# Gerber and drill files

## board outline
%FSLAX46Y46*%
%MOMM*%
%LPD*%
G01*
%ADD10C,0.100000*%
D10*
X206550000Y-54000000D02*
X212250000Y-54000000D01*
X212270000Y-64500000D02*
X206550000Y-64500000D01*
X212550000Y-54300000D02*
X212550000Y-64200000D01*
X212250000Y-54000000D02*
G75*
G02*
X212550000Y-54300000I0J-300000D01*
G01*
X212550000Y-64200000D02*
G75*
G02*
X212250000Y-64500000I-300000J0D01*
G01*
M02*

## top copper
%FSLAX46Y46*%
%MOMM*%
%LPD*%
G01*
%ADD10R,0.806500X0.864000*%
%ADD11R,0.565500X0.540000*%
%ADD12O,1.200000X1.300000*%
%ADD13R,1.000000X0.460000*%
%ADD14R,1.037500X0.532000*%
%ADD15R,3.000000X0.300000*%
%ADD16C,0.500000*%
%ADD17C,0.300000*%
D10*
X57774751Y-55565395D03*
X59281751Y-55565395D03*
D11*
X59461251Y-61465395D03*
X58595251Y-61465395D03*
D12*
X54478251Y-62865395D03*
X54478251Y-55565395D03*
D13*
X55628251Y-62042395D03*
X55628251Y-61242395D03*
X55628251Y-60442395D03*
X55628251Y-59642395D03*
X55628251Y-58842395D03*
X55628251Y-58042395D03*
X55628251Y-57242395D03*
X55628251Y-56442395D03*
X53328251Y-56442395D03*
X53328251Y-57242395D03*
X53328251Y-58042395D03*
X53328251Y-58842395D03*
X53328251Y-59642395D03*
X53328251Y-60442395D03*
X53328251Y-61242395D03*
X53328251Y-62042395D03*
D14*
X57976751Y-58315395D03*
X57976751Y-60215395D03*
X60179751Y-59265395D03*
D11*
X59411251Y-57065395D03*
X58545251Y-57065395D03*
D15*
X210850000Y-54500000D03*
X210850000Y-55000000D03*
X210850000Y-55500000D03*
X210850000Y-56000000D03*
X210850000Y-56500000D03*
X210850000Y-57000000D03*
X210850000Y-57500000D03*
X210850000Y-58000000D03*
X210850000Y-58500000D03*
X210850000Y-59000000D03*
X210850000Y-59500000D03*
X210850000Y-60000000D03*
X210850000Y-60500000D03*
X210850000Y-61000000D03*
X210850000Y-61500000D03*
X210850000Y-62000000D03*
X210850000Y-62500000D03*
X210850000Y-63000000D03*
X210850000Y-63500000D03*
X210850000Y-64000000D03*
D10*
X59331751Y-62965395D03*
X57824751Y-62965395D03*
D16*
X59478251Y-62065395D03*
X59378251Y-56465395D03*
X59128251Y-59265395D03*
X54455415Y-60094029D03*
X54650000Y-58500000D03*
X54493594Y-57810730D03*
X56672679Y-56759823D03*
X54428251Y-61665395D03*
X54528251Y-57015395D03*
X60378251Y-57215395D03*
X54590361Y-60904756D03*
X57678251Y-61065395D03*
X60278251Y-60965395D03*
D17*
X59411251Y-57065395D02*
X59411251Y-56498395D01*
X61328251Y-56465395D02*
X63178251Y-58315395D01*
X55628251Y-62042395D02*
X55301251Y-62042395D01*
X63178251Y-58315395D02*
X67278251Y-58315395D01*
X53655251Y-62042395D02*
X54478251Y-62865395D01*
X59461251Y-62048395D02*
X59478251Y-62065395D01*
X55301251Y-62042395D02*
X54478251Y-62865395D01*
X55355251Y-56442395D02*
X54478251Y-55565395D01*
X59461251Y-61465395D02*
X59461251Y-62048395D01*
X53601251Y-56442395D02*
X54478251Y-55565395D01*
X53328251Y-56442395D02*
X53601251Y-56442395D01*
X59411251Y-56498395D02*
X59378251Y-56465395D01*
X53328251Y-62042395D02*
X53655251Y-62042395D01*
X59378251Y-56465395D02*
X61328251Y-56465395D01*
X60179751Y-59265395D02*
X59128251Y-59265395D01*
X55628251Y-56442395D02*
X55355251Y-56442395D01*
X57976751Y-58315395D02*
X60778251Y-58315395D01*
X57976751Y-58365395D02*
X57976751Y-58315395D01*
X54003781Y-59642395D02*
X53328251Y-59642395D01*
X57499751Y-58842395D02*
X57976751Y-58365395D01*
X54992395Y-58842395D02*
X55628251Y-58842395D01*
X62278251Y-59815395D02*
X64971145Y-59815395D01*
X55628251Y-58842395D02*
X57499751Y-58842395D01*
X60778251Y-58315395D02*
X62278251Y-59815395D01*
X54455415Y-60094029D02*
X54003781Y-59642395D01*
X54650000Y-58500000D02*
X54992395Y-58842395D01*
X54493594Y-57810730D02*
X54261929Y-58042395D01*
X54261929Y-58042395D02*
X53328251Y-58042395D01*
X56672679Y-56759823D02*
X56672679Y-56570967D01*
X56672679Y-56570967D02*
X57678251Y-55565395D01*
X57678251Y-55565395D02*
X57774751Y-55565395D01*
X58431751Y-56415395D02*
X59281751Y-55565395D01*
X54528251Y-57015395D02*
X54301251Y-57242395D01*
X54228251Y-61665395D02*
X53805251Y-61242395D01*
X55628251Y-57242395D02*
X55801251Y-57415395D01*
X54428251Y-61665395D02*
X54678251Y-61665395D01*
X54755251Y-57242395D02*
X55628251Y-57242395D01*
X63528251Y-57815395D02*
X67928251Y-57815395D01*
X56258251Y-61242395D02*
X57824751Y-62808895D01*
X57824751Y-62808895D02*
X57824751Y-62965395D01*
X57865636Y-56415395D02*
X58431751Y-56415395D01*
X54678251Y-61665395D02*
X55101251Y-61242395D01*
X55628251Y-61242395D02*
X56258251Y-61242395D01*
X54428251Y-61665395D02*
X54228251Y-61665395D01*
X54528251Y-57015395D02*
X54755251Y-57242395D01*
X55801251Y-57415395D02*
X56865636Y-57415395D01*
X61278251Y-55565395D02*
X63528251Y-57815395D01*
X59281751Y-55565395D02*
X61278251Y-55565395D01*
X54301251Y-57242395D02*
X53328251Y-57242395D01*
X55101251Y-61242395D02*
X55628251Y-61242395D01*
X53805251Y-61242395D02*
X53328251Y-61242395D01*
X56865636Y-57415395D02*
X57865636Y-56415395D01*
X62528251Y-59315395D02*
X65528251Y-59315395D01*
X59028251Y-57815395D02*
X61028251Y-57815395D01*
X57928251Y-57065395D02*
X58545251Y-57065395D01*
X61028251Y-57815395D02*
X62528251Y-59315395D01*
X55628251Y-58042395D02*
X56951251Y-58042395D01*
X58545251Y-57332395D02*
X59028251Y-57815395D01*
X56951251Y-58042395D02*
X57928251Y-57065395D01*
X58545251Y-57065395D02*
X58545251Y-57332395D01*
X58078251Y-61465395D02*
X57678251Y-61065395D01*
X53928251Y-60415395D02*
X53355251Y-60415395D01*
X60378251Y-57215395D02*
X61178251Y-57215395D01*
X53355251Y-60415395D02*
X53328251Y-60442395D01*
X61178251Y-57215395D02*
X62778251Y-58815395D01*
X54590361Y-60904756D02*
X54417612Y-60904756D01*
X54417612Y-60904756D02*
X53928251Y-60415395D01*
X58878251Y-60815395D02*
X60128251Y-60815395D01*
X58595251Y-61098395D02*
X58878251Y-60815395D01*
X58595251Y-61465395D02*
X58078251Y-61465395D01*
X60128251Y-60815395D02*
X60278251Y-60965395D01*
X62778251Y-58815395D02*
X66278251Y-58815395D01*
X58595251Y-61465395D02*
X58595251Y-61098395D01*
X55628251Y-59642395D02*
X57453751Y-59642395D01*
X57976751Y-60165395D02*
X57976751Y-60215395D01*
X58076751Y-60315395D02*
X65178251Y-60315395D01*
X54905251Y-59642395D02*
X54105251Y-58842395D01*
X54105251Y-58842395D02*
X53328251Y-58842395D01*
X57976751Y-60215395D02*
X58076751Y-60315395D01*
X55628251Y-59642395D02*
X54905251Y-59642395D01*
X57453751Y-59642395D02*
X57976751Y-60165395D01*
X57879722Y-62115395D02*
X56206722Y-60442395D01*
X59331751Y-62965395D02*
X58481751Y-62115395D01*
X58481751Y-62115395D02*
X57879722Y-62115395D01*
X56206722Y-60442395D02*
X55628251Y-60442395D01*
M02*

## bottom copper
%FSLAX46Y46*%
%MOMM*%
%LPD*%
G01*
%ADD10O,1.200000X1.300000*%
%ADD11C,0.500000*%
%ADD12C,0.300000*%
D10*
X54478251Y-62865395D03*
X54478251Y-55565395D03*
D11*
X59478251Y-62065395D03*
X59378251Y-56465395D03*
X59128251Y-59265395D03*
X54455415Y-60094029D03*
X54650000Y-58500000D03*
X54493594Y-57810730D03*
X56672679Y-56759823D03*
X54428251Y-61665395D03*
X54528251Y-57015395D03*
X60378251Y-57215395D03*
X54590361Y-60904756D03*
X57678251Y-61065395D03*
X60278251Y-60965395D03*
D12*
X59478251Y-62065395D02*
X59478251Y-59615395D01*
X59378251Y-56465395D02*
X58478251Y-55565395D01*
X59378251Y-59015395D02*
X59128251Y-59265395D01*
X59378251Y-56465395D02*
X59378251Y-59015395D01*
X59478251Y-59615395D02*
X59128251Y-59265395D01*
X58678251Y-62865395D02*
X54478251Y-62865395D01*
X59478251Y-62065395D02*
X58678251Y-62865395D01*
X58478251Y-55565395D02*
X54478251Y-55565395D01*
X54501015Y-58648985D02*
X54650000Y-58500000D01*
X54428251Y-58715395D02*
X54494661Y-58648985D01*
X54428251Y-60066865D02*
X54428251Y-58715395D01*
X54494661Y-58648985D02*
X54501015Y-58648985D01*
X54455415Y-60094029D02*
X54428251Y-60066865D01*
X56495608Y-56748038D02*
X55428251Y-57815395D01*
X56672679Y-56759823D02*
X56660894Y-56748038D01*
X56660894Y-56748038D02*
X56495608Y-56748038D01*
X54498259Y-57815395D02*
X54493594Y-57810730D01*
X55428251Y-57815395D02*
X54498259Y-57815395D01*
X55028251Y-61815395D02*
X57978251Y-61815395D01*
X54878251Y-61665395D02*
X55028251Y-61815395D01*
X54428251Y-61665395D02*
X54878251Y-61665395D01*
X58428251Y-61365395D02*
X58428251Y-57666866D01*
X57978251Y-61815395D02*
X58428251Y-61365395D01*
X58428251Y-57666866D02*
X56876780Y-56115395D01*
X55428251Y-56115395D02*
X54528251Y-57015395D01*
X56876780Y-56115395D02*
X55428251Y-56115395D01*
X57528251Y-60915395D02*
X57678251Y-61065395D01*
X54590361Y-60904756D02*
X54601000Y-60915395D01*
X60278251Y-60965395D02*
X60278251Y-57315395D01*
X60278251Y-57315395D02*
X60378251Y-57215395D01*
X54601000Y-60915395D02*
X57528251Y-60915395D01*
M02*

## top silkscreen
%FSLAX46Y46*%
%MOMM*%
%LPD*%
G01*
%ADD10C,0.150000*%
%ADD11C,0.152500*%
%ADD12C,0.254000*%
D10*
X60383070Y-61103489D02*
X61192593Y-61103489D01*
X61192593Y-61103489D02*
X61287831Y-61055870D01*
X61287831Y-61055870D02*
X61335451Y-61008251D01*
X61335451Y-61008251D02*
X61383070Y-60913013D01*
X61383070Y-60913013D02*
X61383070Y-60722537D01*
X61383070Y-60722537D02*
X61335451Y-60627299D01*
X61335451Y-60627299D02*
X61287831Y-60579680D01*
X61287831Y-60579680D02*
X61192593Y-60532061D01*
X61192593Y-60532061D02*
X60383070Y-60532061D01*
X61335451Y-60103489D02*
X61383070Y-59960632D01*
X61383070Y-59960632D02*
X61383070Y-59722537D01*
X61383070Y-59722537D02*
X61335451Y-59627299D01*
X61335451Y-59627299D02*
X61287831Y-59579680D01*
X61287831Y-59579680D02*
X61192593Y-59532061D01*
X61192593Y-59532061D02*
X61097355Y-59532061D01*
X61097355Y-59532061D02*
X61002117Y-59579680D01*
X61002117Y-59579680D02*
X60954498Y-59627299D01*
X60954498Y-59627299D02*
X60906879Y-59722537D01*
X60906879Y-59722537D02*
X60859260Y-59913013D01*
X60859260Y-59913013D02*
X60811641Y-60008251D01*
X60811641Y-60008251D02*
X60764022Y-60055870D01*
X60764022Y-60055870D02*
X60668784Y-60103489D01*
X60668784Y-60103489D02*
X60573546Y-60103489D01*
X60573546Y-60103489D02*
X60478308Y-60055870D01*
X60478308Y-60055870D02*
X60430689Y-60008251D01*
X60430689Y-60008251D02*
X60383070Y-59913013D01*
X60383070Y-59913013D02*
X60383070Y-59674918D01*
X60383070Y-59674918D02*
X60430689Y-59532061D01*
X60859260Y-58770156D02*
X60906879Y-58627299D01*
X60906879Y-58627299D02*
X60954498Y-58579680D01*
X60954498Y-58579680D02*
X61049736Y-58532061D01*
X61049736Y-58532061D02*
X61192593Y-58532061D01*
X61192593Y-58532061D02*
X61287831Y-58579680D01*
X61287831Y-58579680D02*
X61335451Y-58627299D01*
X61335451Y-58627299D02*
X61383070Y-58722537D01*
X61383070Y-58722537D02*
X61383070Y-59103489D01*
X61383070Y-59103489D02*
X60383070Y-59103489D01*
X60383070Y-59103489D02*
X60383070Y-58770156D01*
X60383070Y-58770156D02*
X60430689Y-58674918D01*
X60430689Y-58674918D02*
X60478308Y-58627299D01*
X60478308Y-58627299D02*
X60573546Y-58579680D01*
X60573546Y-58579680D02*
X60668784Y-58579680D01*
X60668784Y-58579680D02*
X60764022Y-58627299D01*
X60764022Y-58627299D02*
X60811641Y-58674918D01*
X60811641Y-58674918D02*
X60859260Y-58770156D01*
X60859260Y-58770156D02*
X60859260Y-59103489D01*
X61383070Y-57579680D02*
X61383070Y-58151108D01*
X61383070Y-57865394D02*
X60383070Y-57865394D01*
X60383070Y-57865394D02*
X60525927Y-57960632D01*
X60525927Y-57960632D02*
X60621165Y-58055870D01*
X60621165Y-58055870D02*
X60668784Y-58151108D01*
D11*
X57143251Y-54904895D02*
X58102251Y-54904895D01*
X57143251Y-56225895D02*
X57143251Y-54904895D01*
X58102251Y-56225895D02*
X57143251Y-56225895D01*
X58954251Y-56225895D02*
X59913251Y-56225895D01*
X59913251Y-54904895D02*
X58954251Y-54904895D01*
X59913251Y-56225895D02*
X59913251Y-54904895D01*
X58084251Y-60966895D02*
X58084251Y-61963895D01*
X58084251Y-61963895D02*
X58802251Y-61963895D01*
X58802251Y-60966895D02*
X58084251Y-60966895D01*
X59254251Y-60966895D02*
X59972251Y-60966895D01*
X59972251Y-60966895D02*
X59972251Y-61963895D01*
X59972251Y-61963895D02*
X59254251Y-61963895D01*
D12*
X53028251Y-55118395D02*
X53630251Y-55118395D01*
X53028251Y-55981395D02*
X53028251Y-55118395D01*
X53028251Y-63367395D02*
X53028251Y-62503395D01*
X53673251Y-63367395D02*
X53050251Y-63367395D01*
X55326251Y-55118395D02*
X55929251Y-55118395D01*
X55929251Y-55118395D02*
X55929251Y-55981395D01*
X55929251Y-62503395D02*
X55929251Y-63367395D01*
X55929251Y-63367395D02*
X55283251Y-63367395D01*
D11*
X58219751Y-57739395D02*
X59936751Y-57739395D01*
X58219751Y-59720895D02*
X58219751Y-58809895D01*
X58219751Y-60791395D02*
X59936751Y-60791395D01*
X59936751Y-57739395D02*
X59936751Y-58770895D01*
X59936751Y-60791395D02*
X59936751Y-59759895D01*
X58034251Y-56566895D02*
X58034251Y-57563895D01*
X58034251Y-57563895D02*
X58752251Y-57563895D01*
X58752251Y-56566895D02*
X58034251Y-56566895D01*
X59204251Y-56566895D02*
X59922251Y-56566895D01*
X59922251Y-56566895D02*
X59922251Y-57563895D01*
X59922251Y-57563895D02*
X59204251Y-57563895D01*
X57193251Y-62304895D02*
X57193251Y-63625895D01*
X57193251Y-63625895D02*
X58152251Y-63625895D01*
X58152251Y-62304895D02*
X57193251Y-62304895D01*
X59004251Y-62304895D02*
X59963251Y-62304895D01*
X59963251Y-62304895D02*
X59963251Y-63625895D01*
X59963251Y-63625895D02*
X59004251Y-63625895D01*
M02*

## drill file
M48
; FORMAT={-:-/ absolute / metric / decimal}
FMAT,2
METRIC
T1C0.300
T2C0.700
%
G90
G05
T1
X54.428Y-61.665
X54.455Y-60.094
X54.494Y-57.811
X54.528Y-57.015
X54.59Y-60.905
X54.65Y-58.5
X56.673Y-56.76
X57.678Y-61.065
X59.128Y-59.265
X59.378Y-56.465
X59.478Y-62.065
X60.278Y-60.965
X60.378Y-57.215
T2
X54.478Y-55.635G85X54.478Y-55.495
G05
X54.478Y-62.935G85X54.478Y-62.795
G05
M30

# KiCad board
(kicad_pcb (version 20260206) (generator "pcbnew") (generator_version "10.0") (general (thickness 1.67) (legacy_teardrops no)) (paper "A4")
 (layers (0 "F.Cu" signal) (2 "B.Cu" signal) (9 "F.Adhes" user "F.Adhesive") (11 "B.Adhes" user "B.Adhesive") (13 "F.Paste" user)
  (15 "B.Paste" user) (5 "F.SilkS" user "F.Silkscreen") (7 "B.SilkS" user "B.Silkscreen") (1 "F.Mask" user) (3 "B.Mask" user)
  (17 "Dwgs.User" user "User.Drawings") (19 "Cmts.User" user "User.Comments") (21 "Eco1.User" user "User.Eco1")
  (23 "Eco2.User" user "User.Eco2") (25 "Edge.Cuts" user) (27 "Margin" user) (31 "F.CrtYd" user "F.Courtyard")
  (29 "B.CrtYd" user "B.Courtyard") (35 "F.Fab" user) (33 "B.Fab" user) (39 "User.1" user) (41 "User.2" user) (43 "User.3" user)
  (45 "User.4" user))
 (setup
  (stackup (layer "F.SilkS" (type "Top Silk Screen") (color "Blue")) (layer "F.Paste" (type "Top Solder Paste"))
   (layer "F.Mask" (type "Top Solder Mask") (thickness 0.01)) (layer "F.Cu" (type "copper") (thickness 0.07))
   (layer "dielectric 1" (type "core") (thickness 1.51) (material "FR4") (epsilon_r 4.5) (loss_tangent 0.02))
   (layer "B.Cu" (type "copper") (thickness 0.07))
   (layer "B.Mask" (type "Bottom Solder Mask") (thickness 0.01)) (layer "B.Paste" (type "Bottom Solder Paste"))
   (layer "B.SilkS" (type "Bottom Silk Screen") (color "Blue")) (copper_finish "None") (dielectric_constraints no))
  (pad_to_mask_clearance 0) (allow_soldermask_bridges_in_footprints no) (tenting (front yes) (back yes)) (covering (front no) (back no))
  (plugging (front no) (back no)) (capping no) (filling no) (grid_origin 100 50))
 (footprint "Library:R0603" (layer "F.Cu") (at 58.528251 55.565395)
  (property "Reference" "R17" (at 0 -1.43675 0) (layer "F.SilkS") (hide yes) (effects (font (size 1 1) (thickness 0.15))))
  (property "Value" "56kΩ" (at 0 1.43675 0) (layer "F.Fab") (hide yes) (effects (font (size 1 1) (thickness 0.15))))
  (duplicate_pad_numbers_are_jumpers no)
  (fp_line (start -1.385 -0.6605) (end -0.426 -0.6605) (stroke (width 0.1525) (type default)) (layer "F.SilkS"))
  (fp_line (start -1.385 0.6605) (end -1.385 -0.6605) (stroke (width 0.1525) (type default)) (layer "F.SilkS"))
  (fp_line (start -0.426 0.6605) (end -1.385 0.6605) (stroke (width 0.1525) (type default)) (layer "F.SilkS"))
  (fp_line (start 0.426 0.6605) (end 1.385 0.6605) (stroke (width 0.1525) (type default)) (layer "F.SilkS"))
  (fp_line (start 1.385 -0.6605) (end 0.426 -0.6605) (stroke (width 0.1525) (type default)) (layer "F.SilkS"))
  (fp_line (start 1.385 0.6605) (end 1.385 -0.6605) (stroke (width 0.1525) (type default)) (layer "F.SilkS"))
  (pad "1" smd rect (at -0.7535 0) (size 0.8065 0.864) (layers "F.Cu" "F.Mask" "F.Paste") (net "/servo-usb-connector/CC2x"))
  (pad "2" smd rect (at 0.7535 0) (size 0.8065 0.864) (layers "F.Cu" "F.Mask" "F.Paste") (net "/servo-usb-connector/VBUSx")))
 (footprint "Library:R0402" (layer "F.Cu") (at 59.028251 61.465395 180)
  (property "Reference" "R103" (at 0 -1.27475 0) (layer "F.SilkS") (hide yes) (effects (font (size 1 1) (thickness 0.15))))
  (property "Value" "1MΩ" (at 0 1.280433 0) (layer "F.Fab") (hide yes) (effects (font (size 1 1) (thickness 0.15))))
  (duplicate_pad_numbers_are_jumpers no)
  (fp_line (start 0.944 0.4985) (end 0.944 -0.4985) (stroke (width 0.1525) (type default)) (layer "F.SilkS"))
  (fp_line (start 0.944 -0.4985) (end 0.226 -0.4985) (stroke (width 0.1525) (type default)) (layer "F.SilkS"))
  (fp_line (start 0.226 0.4985) (end 0.944 0.4985) (stroke (width 0.1525) (type default)) (layer "F.SilkS"))
  (fp_line (start -0.226 0.4985) (end -0.944 0.4985) (stroke (width 0.1525) (type default)) (layer "F.SilkS"))
  (fp_line (start -0.944 0.4985) (end -0.944 -0.4985) (stroke (width 0.1525) (type default)) (layer "F.SilkS"))
  (fp_line (start -0.944 -0.4985) (end -0.226 -0.4985) (stroke (width 0.1525) (type default)) (layer "F.SilkS"))
  (pad "1" smd rect (at -0.433 0 180) (size 0.5655 0.54) (layers "F.Cu" "F.Mask" "F.Paste") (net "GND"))
  (pad "2" smd rect (at 0.433 0 180) (size 0.5655 0.54) (layers "F.Cu" "F.Mask" "F.Paste") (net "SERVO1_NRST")))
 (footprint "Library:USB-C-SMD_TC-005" (layer "F.Cu") (at 54.478251 59.215395 90)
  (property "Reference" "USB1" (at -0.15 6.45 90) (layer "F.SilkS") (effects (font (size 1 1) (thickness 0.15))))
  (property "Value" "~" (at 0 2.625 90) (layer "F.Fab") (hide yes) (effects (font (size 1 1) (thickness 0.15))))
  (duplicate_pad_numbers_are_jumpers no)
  (fp_line (start 4.097 -1.45) (end 4.097 -0.848) (stroke (width 0.254) (type default)) (layer "F.SilkS"))
  (fp_line (start 3.234 -1.45) (end 4.097 -1.45) (stroke (width 0.254) (type default)) (layer "F.SilkS"))
  (fp_line (start -4.152 -1.45) (end -3.288 -1.45) (stroke (width 0.254) (type default)) (layer "F.SilkS"))
  (fp_line (start -4.152 -0.805) (end -4.152 -1.428) (stroke (width 0.254) (type default)) (layer "F.SilkS"))
  (fp_line (start 4.097 0.848) (end 4.097 1.451) (stroke (width 0.254) (type default)) (layer "F.SilkS"))
  (fp_line (start 4.097 1.451) (end 3.234 1.451) (stroke (width 0.254) (type default)) (layer "F.SilkS"))
  (fp_line (start -3.288 1.451) (end -4.152 1.451) (stroke (width 0.254) (type default)) (layer "F.SilkS"))
  (fp_line (start -4.152 1.451) (end -4.152 0.805) (stroke (width 0.254) (type default)) (layer "F.SilkS"))
  (pad "1" thru_hole oval (at -3.65 0 90) (size 1.3 1.2) (drill oval 0.84 0.7) (layers "*.Cu" "*.Mask") (remove_unused_layers no)
   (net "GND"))
  (pad "2" thru_hole oval (at 3.65 0 90) (size 1.3 1.2) (drill oval 0.84 0.7) (layers "*.Cu" "*.Mask") (remove_unused_layers no) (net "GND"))
  (pad "A1" smd rect (at -2.827 1.15 90) (size 0.46 1) (layers "F.Cu" "F.Mask" "F.Paste") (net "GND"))
  (pad "A4" smd rect (at -2.027 1.15 90) (size 0.46 1) (layers "F.Cu" "F.Mask" "F.Paste") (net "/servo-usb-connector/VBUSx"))
  (pad "A5" smd rect (at -1.227 1.15 90) (size 0.46 1) (layers "F.Cu" "F.Mask" "F.Paste") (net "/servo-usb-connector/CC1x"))
  (pad "A6" smd rect (at -0.427 1.15 90) (size 0.46 1) (layers "F.Cu" "F.Mask" "F.Paste") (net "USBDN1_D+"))
  (pad "A7" smd rect (at 0.373 1.15 90) (size 0.46 1) (layers "F.Cu" "F.Mask" "F.Paste") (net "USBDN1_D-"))
  (pad "A8" smd rect (at 1.173 1.15 90) (size 0.46 1) (layers "F.Cu" "F.Mask" "F.Paste") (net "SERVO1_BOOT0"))
  (pad "A9" smd rect (at 1.973 1.15 90) (size 0.46 1) (layers "F.Cu" "F.Mask" "F.Paste") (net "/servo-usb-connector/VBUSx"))
  (pad "A12" smd rect (at 2.773 1.15 90) (size 0.46 1) (layers "F.Cu" "F.Mask" "F.Paste") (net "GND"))
  (pad "B1" smd rect (at 2.773 -1.15 90) (size 0.46 1) (layers "F.Cu" "F.Mask" "F.Paste") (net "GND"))
  (pad "B4" smd rect (at 1.973 -1.15 90) (size 0.46 1) (layers "F.Cu" "F.Mask" "F.Paste") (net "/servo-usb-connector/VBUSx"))
  (pad "B5" smd rect (at 1.173 -1.15 90) (size 0.46 1) (layers "F.Cu" "F.Mask" "F.Paste") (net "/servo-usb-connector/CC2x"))
  (pad "B6" smd rect (at 0.373 -1.15 90) (size 0.46 1) (layers "F.Cu" "F.Mask" "F.Paste") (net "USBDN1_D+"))
  (pad "B7" smd rect (at -0.427 -1.15 90) (size 0.46 1) (layers "F.Cu" "F.Mask" "F.Paste") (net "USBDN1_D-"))
  (pad "B8" smd rect (at -1.227 -1.15 90) (size 0.46 1) (layers "F.Cu" "F.Mask" "F.Paste") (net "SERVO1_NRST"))
  (pad "B9" smd rect (at -2.027 -1.15 90) (size 0.46 1) (layers "F.Cu" "F.Mask" "F.Paste") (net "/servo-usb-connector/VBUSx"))
  (pad "B12" smd rect (at -2.827 -1.15 90) (size 0.46 1) (layers "F.Cu" "F.Mask" "F.Paste") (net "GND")))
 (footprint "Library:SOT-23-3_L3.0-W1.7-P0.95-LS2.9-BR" (layer "F.Cu") (at 59.078251 59.265395)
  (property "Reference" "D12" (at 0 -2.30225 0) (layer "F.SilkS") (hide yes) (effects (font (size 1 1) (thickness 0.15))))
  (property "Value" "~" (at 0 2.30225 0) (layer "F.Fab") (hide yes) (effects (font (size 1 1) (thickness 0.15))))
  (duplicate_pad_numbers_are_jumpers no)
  (fp_line (start -0.8585 -1.526) (end 0.8585 -1.526) (stroke (width 0.1525) (type default)) (layer "F.SilkS"))
  (fp_line (start -0.8585 0.4555) (end -0.8585 -0.4555) (stroke (width 0.1525) (type default)) (layer "F.SilkS"))
  (fp_line (start -0.8585 1.526) (end 0.8585 1.526) (stroke (width 0.1525) (type default)) (layer "F.SilkS"))
  (fp_line (start 0.8585 -1.526) (end 0.8585 -0.4945) (stroke (width 0.1525) (type default)) (layer "F.SilkS"))
  (fp_line (start 0.8585 1.526) (end 0.8585 0.4945) (stroke (width 0.1525) (type default)) (layer "F.SilkS"))
  (pad "1" smd rect (at -1.1015 -0.95 180) (size 1.0375 0.532) (layers "F.Cu" "F.Mask" "F.Paste") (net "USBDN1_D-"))
  (pad "2" smd rect (at -1.1015 0.95 180) (size 1.0375 0.532) (layers "F.Cu" "F.Mask" "F.Paste") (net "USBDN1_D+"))
  (pad "3" smd rect (at 1.1015 0 180) (size 1.0375 0.532) (layers "F.Cu" "F.Mask" "F.Paste") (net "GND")))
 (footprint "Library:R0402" (layer "F.Cu") (at 58.978251 57.065395 180)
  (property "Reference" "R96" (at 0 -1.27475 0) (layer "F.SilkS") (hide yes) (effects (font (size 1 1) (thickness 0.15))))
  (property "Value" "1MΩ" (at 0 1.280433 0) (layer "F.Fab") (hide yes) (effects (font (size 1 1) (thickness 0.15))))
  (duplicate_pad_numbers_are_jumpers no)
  (fp_line (start 0.944 0.4985) (end 0.944 -0.4985) (stroke (width 0.1525) (type default)) (layer "F.SilkS"))
  (fp_line (start 0.944 -0.4985) (end 0.226 -0.4985) (stroke (width 0.1525) (type default)) (layer "F.SilkS"))
  (fp_line (start 0.226 0.4985) (end 0.944 0.4985) (stroke (width 0.1525) (type default)) (layer "F.SilkS"))
  (fp_line (start -0.226 0.4985) (end -0.944 0.4985) (stroke (width 0.1525) (type default)) (layer "F.SilkS"))
  (fp_line (start -0.944 0.4985) (end -0.944 -0.4985) (stroke (width 0.1525) (type default)) (layer "F.SilkS"))
  (fp_line (start -0.944 -0.4985) (end -0.226 -0.4985) (stroke (width 0.1525) (type default)) (layer "F.SilkS"))
  (pad "1" smd rect (at -0.433 0 180) (size 0.5655 0.54) (layers "F.Cu" "F.Mask" "F.Paste") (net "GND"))
  (pad "2" smd rect (at 0.433 0 180) (size 0.5655 0.54) (layers "F.Cu" "F.Mask" "F.Paste") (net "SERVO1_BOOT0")))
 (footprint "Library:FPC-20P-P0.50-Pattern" (layer "F.Cu") (at 210.85 59.25 -90)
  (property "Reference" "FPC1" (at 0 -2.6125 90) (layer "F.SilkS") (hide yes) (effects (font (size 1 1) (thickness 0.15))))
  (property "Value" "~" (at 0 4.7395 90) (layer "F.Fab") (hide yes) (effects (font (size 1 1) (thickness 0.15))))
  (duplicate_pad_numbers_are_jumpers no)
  (fp_line (start -5.25 4.3) (end -5.25 -1.4) (stroke (width 0.1) (type solid)) (layer "Edge.Cuts"))
  (fp_line (start 5.25 -1.42) (end 5.25 4.3) (stroke (width 0.1) (type solid)) (layer "Edge.Cuts"))
  (fp_line (start -4.95 -1.7) (end 4.95 -1.7) (stroke (width 0.1) (type solid)) (layer "Edge.Cuts"))
  (fp_arc (start -5.25 -1.4) (mid -5.162132 -1.612132) (end -4.95 -1.7) (stroke (width 0.1) (type solid)) (layer "Edge.Cuts"))
  (fp_arc (start 4.95 -1.7) (mid 5.162132 -1.612132) (end 5.25 -1.4) (stroke (width 0.1) (type solid)) (layer "Edge.Cuts"))
  (pad "1" smd rect (at -4.75 0 270) (size 0.3 3) (layers "F.Cu" "F.Mask") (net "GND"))
  (pad "2" smd rect (at -4.25 0 270) (size 0.3 3) (layers "F.Cu" "F.Mask") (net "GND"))
  (pad "3" smd rect (at -3.75 0 270) (size 0.3 3) (layers "F.Cu" "F.Mask") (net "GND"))
  (pad "4" smd rect (at -3.25 0 270) (size 0.3 3) (layers "F.Cu" "F.Mask") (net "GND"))
  (pad "5" smd rect (at -2.75 0 270) (size 0.3 3) (layers "F.Cu" "F.Mask") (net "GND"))
  (pad "6" smd rect (at -2.25 0 270) (size 0.3 3) (layers "F.Cu" "F.Mask") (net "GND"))
  (pad "7" smd rect (at -1.75 0 270) (size 0.3 3) (layers "F.Cu" "F.Mask") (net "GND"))
  (pad "8" smd rect (at -1.25 0 270) (size 0.3 3) (layers "F.Cu" "F.Mask") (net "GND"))
  (pad "9" smd rect (at -0.75 0 270) (size 0.3 3) (layers "F.Cu" "F.Mask") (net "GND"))
  (pad "10" smd rect (at -0.25 0 270) (size 0.3 3) (layers "F.Cu" "F.Mask") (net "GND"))
  (pad "11" smd rect (at 0.25 0 270) (size 0.3 3) (layers "F.Cu" "F.Mask") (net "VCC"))
  (pad "12" smd rect (at 0.75 0 270) (size 0.3 3) (layers "F.Cu" "F.Mask") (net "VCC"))
  (pad "13" smd rect (at 1.25 0 270) (size 0.3 3) (layers "F.Cu" "F.Mask") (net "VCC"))
  (pad "14" smd rect (at 1.75 0 270) (size 0.3 3) (layers "F.Cu" "F.Mask") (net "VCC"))
  (pad "15" smd rect (at 2.25 0 270) (size 0.3 3) (layers "F.Cu" "F.Mask") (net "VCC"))
  (pad "16" smd rect (at 2.75 0 270) (size 0.3 3) (layers "F.Cu" "F.Mask") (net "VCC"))
  (pad "17" smd rect (at 3.25 0 270) (size 0.3 3) (layers "F.Cu" "F.Mask") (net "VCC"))
  (pad "18" smd rect (at 3.75 0 270) (size 0.3 3) (layers "F.Cu" "F.Mask") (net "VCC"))
  (pad "19" smd rect (at 4.25 0 270) (size 0.3 3) (layers "F.Cu" "F.Mask") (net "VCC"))
  (pad "20" smd rect (at 4.75 0 270) (size 0.3 3) (layers "F.Cu" "F.Mask") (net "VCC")))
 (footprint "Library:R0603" (layer "F.Cu") (at 58.578251 62.965395 180)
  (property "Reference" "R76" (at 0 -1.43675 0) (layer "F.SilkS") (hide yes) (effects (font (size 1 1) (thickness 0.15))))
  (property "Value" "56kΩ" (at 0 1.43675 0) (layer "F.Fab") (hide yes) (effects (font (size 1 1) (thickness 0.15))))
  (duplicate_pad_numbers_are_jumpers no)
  (fp_line (start 1.385 0.6605) (end 1.385 -0.6605) (stroke (width 0.1525) (type default)) (layer "F.SilkS"))
  (fp_line (start 1.385 -0.6605) (end 0.426 -0.6605) (stroke (width 0.1525) (type default)) (layer "F.SilkS"))
  (fp_line (start 0.426 0.6605) (end 1.385 0.6605) (stroke (width 0.1525) (type default)) (layer "F.SilkS"))
  (fp_line (start -0.426 0.6605) (end -1.385 0.6605) (stroke (width 0.1525) (type default)) (layer "F.SilkS"))
  (fp_line (start -1.385 0.6605) (end -1.385 -0.6605) (stroke (width 0.1525) (type default)) (layer "F.SilkS"))
  (fp_line (start -1.385 -0.6605) (end -0.426 -0.6605) (stroke (width 0.1525) (type default)) (layer "F.SilkS"))
  (pad "1" smd rect (at -0.7535 0 180) (size 0.8065 0.864) (layers "F.Cu" "F.Mask" "F.Paste") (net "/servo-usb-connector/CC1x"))
  (pad "2" smd rect (at 0.7535 0 180) (size 0.8065 0.864) (layers "F.Cu" "F.Mask" "F.Paste") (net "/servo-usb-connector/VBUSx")))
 (segment (start 59.411251 57.065395) (end 59.411251 56.498395) (width 0.3) (layer "F.Cu") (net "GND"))
 (segment (start 61.328251 56.465395) (end 63.178251 58.315395) (width 0.3) (layer "F.Cu") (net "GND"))
 (segment (start 55.628251 62.042395) (end 55.301251 62.042395) (width 0.3) (layer "F.Cu") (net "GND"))
 (segment (start 63.178251 58.315395) (end 67.278251 58.315395) (width 0.3) (layer "F.Cu") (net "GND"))
 (segment (start 53.655251 62.042395) (end 54.478251 62.865395) (width 0.3) (layer "F.Cu") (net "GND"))
 (segment (start 59.461251 62.048395) (end 59.478251 62.065395) (width 0.3) (layer "F.Cu") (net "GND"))
 (segment (start 55.301251 62.042395) (end 54.478251 62.865395) (width 0.3) (layer "F.Cu") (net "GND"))
 (segment (start 55.355251 56.442395) (end 54.478251 55.565395) (width 0.3) (layer "F.Cu") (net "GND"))
 (segment (start 59.461251 61.465395) (end 59.461251 62.048395) (width 0.3) (layer "F.Cu") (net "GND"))
 (segment (start 53.601251 56.442395) (end 54.478251 55.565395) (width 0.3) (layer "F.Cu") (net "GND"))
 (segment (start 53.328251 56.442395) (end 53.601251 56.442395) (width 0.3) (layer "F.Cu") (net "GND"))
 (segment (start 59.411251 56.498395) (end 59.378251 56.465395) (width 0.3) (layer "F.Cu") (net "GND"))
 (segment (start 53.328251 62.042395) (end 53.655251 62.042395) (width 0.3) (layer "F.Cu") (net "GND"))
 (segment (start 59.378251 56.465395) (end 61.328251 56.465395) (width 0.3) (layer "F.Cu") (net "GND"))
 (segment (start 60.179751 59.265395) (end 59.128251 59.265395) (width 0.3) (layer "F.Cu") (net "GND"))
 (segment (start 55.628251 56.442395) (end 55.355251 56.442395) (width 0.3) (layer "F.Cu") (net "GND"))
 (via (at 59.478251 62.065395) (size 0.5) (drill 0.3) (layers "F.Cu" "B.Cu") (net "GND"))
 (via (at 59.378251 56.465395) (size 0.5) (drill 0.3) (layers "F.Cu" "B.Cu") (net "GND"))
 (via (at 59.128251 59.265395) (size 0.5) (drill 0.3) (layers "F.Cu" "B.Cu") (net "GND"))
 (segment (start 59.478251 62.065395) (end 59.478251 59.615395) (width 0.3) (layer "B.Cu") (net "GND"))
 (segment (start 59.378251 56.465395) (end 58.478251 55.565395) (width 0.3) (layer "B.Cu") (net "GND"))
 (segment (start 59.378251 59.015395) (end 59.128251 59.265395) (width 0.3) (layer "B.Cu") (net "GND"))
 (segment (start 59.378251 56.465395) (end 59.378251 59.015395) (width 0.3) (layer "B.Cu") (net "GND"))
 (segment (start 59.478251 59.615395) (end 59.128251 59.265395) (width 0.3) (layer "B.Cu") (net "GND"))
 (segment (start 58.678251 62.865395) (end 54.478251 62.865395) (width 0.3) (layer "B.Cu") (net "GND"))
 (segment (start 59.478251 62.065395) (end 58.678251 62.865395) (width 0.3) (layer "B.Cu") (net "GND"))
 (segment (start 58.478251 55.565395) (end 54.478251 55.565395) (width 0.3) (layer "B.Cu") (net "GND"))
 (segment (start 57.976751 58.315395) (end 60.778251 58.315395) (width 0.3) (layer "F.Cu") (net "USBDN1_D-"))
 (segment (start 57.976751 58.365395) (end 57.976751 58.315395) (width 0.3) (layer "F.Cu") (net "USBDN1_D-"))
 (segment (start 54.003781 59.642395) (end 53.328251 59.642395) (width 0.3) (layer "F.Cu") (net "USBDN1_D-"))
 (segment (start 57.499751 58.842395) (end 57.976751 58.365395) (width 0.3) (layer "F.Cu") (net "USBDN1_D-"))
 (segment (start 54.992395 58.842395) (end 55.628251 58.842395) (width 0.3) (layer "F.Cu") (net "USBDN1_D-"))
 (segment (start 62.278251 59.815395) (end 64.971145 59.815395) (width 0.3) (layer "F.Cu") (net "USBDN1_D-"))
 (segment (start 55.628251 58.842395) (end 57.499751 58.842395) (width 0.3) (layer "F.Cu") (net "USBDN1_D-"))
 (segment (start 60.778251 58.315395) (end 62.278251 59.815395) (width 0.3) (layer "F.Cu") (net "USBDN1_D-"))
 (segment (start 54.455415 60.094029) (end 54.003781 59.642395) (width 0.3) (layer "F.Cu") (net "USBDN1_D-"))
 (segment (start 54.65 58.5) (end 54.992395 58.842395) (width 0.3) (layer "F.Cu") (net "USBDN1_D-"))
 (via (at 54.455415 60.094029) (size 0.5) (drill 0.3) (layers "F.Cu" "B.Cu") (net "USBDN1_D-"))
 (via (at 54.65 58.5) (size 0.5) (drill 0.3) (layers "F.Cu" "B.Cu") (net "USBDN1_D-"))
 (segment (start 54.501015 58.648985) (end 54.65 58.5) (width 0.3) (layer "B.Cu") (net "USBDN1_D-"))
 (segment (start 54.428251 58.715395) (end 54.494661 58.648985) (width 0.3) (layer "B.Cu") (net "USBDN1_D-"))
 (segment (start 54.428251 60.066865) (end 54.428251 58.715395) (width 0.3) (layer "B.Cu") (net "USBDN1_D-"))
 (segment (start 54.494661 58.648985) (end 54.501015 58.648985) (width 0.3) (layer "B.Cu") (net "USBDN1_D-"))
 (segment (start 54.455415 60.094029) (end 54.428251 60.066865) (width 0.3) (layer "B.Cu") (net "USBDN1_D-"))
 (segment (start 54.493594 57.81073) (end 54.261929 58.042395) (width 0.3) (layer "F.Cu") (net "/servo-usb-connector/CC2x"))
 (segment (start 54.261929 58.042395) (end 53.328251 58.042395) (width 0.3) (layer "F.Cu") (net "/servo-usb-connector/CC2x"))
 (segment (start 56.672679 56.759823) (end 56.672679 56.570967) (width 0.3) (layer "F.Cu") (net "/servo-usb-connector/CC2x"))
 (segment (start 56.672679 56.570967) (end 57.678251 55.565395) (width 0.3) (layer "F.Cu") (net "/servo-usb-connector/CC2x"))
 (segment (start 57.678251 55.565395) (end 57.774751 55.565395) (width 0.3) (layer "F.Cu") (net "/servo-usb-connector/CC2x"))
 (via (at 54.493594 57.81073) (size 0.5) (drill 0.3) (layers "F.Cu" "B.Cu") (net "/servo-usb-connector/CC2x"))
 (via (at 56.672679 56.759823) (size 0.5) (drill 0.3) (layers "F.Cu" "B.Cu") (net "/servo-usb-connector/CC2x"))
 (segment (start 56.495608 56.748038) (end 55.428251 57.815395) (width 0.3) (layer "B.Cu") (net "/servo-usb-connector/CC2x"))
 (segment (start 56.672679 56.759823) (end 56.660894 56.748038) (width 0.3) (layer "B.Cu") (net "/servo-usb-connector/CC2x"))
 (segment (start 56.660894 56.748038) (end 56.495608 56.748038) (width 0.3) (layer "B.Cu") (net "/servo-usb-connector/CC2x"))
 (segment (start 54.498259 57.815395) (end 54.493594 57.81073) (width 0.3) (layer "B.Cu") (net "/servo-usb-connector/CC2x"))
 (segment (start 55.428251 57.815395) (end 54.498259 57.815395) (width 0.3) (layer "B.Cu") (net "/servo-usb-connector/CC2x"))
 (segment (start 58.431751 56.415395) (end 59.281751 55.565395) (width 0.3) (layer "F.Cu") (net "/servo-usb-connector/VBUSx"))
 (segment (start 54.528251 57.015395) (end 54.301251 57.242395) (width 0.3) (layer "F.Cu") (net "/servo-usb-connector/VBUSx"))
 (segment (start 54.228251 61.665395) (end 53.805251 61.242395) (width 0.3) (layer "F.Cu") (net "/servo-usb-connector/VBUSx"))
 (segment (start 55.628251 57.242395) (end 55.801251 57.415395) (width 0.3) (layer "F.Cu") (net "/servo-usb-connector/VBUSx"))
 (segment (start 54.428251 61.665395) (end 54.678251 61.665395) (width 0.3) (layer "F.Cu") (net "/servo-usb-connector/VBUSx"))
 (segment (start 54.755251 57.242395) (end 55.628251 57.242395) (width 0.3) (layer "F.Cu") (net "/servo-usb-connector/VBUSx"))
 (segment (start 63.528251 57.815395) (end 67.928251 57.815395) (width 0.3) (layer "F.Cu") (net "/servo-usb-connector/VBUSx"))
 (segment (start 56.258251 61.242395) (end 57.824751 62.808895) (width 0.3) (layer "F.Cu") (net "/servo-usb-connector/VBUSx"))
 (segment (start 57.824751 62.808895) (end 57.824751 62.965395) (width 0.3) (layer "F.Cu") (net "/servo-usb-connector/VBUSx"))
 (segment (start 57.865636 56.415395) (end 58.431751 56.415395) (width 0.3) (layer "F.Cu") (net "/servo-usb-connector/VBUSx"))
 (segment (start 54.678251 61.665395) (end 55.101251 61.242395) (width 0.3) (layer "F.Cu") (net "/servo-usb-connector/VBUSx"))
 (segment (start 55.628251 61.242395) (end 56.258251 61.242395) (width 0.3) (layer "F.Cu") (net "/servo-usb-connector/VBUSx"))
 (segment (start 54.428251 61.665395) (end 54.228251 61.665395) (width 0.3) (layer "F.Cu") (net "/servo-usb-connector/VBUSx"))
 (segment (start 54.528251 57.015395) (end 54.755251 57.242395) (width 0.3) (layer "F.Cu") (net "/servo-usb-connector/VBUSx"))
 (segment (start 55.801251 57.415395) (end 56.865636 57.415395) (width 0.3) (layer "F.Cu") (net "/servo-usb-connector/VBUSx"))
 (segment (start 61.278251 55.565395) (end 63.528251 57.815395) (width 0.3) (layer "F.Cu") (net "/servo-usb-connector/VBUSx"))
 (segment (start 59.281751 55.565395) (end 61.278251 55.565395) (width 0.3) (layer "F.Cu") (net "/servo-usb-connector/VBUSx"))
 (segment (start 54.301251 57.242395) (end 53.328251 57.242395) (width 0.3) (layer "F.Cu") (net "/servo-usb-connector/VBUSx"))
 (segment (start 55.101251 61.242395) (end 55.628251 61.242395) (width 0.3) (layer "F.Cu") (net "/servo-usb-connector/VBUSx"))
 (segment (start 53.805251 61.242395) (end 53.328251 61.242395) (width 0.3) (layer "F.Cu") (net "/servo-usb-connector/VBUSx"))
 (segment (start 56.865636 57.415395) (end 57.865636 56.415395) (width 0.3) (layer "F.Cu") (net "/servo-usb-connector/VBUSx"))
 (via (at 54.428251 61.665395) (size 0.5) (drill 0.3) (layers "F.Cu" "B.Cu") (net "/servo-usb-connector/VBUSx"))
 (via (at 54.528251 57.015395) (size 0.5) (drill 0.3) (layers "F.Cu" "B.Cu") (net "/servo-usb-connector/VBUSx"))
 (segment (start 55.028251 61.815395) (end 57.978251 61.815395) (width 0.3) (layer "B.Cu") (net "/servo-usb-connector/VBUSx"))
 (segment (start 54.878251 61.665395) (end 55.028251 61.815395) (width 0.3) (layer "B.Cu") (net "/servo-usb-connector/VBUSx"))
 (segment (start 54.428251 61.665395) (end 54.878251 61.665395) (width 0.3) (layer "B.Cu") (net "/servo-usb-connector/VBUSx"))
 (segment (start 58.428251 61.365395) (end 58.428251 57.666866) (width 0.3) (layer "B.Cu") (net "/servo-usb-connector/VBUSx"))
 (segment (start 57.978251 61.815395) (end 58.428251 61.365395) (width 0.3) (layer "B.Cu") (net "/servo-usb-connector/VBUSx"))
 (segment (start 58.428251 57.666866) (end 56.87678 56.115395) (width 0.3) (layer "B.Cu") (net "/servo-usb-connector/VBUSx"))
 (segment (start 55.428251 56.115395) (end 54.528251 57.015395) (width 0.3) (layer "B.Cu") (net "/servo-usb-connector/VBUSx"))
 (segment (start 56.87678 56.115395) (end 55.428251 56.115395) (width 0.3) (layer "B.Cu") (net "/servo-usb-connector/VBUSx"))
 (segment (start 62.528251 59.315395) (end 65.528251 59.315395) (width 0.3) (layer "F.Cu") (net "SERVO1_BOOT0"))
 (segment (start 59.028251 57.815395) (end 61.028251 57.815395) (width 0.3) (layer "F.Cu") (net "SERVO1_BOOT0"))
 (segment (start 57.928251 57.065395) (end 58.545251 57.065395) (width 0.3) (layer "F.Cu") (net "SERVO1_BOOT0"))
 (segment (start 61.028251 57.815395) (end 62.528251 59.315395) (width 0.3) (layer "F.Cu") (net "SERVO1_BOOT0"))
 (segment (start 55.628251 58.042395) (end 56.951251 58.042395) (width 0.3) (layer "F.Cu") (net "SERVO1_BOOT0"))
 (segment (start 58.545251 57.332395) (end 59.028251 57.815395) (width 0.3) (layer "F.Cu") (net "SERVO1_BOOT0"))
 (segment (start 56.951251 58.042395) (end 57.928251 57.065395) (width 0.3) (layer "F.Cu") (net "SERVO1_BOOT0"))
 (segment (start 58.545251 57.065395) (end 58.545251 57.332395) (width 0.3) (layer "F.Cu") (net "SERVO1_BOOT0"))
 (segment (start 58.078251 61.465395) (end 57.678251 61.065395) (width 0.3) (layer "F.Cu") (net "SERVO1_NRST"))
 (segment (start 53.928251 60.415395) (end 53.355251 60.415395) (width 0.3) (layer "F.Cu") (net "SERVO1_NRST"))
 (segment (start 60.378251 57.215395) (end 61.178251 57.215395) (width 0.3) (layer "F.Cu") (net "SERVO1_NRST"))
 (segment (start 53.355251 60.415395) (end 53.328251 60.442395) (width 0.3) (layer "F.Cu") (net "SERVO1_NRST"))
 (segment (start 61.178251 57.215395) (end 62.778251 58.815395) (width 0.3) (layer "F.Cu") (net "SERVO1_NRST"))
 (segment (start 54.590361 60.904756) (end 54.417612 60.904756) (width 0.3) (layer "F.Cu") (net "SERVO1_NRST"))
 (segment (start 54.417612 60.904756) (end 53.928251 60.415395) (width 0.3) (layer "F.Cu") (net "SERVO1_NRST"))
 (segment (start 58.878251 60.815395) (end 60.128251 60.815395) (width 0.3) (layer "F.Cu") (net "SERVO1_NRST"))
 (segment (start 58.595251 61.098395) (end 58.878251 60.815395) (width 0.3) (layer "F.Cu") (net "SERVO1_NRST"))
 (segment (start 58.595251 61.465395) (end 58.078251 61.465395) (width 0.3) (layer "F.Cu") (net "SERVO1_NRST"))
 (segment (start 60.128251 60.815395) (end 60.278251 60.965395) (width 0.3) (layer "F.Cu") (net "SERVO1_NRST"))
 (segment (start 62.778251 58.815395) (end 66.278251 58.815395) (width 0.3) (layer "F.Cu") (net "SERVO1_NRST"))
 (segment (start 58.595251 61.465395) (end 58.595251 61.098395) (width 0.3) (layer "F.Cu") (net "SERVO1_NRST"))
 (via (at 60.378251 57.215395) (size 0.5) (drill 0.3) (layers "F.Cu" "B.Cu") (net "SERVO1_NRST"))
 (via (at 54.590361 60.904756) (size 0.5) (drill 0.3) (layers "F.Cu" "B.Cu") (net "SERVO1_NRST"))
 (via (at 57.678251 61.065395) (size 0.5) (drill 0.3) (layers "F.Cu" "B.Cu") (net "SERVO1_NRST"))
 (via (at 60.278251 60.965395) (size 0.5) (drill 0.3) (layers "F.Cu" "B.Cu") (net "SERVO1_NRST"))
 (segment (start 57.528251 60.915395) (end 57.678251 61.065395) (width 0.3) (layer "B.Cu") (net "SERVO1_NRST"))
 (segment (start 54.590361 60.904756) (end 54.601 60.915395) (width 0.3) (layer "B.Cu") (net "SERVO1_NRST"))
 (segment (start 60.278251 60.965395) (end 60.278251 57.315395) (width 0.3) (layer "B.Cu") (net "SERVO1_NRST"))
 (segment (start 60.278251 57.315395) (end 60.378251 57.215395) (width 0.3) (layer "B.Cu") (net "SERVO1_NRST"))
 (segment (start 54.601 60.915395) (end 57.528251 60.915395) (width 0.3) (layer "B.Cu") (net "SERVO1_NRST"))
 (segment (start 55.628251 59.642395) (end 57.453751 59.642395) (width 0.3) (layer "F.Cu") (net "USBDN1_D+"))
 (segment (start 57.976751 60.165395) (end 57.976751 60.215395) (width 0.3) (layer "F.Cu") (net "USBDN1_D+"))
 (segment (start 58.076751 60.315395) (end 65.178251 60.315395) (width 0.3) (layer "F.Cu") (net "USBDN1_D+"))
 (segment (start 54.905251 59.642395) (end 54.105251 58.842395) (width 0.3) (layer "F.Cu") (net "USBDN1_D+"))
 (segment (start 54.105251 58.842395) (end 53.328251 58.842395) (width 0.3) (layer "F.Cu") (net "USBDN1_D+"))
 (segment (start 57.976751 60.215395) (end 58.076751 60.315395) (width 0.3) (layer "F.Cu") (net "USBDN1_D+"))
 (segment (start 55.628251 59.642395) (end 54.905251 59.642395) (width 0.3) (layer "F.Cu") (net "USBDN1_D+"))
 (segment (start 57.453751 59.642395) (end 57.976751 60.165395) (width 0.3) (layer "F.Cu") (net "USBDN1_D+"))
 (segment (start 57.879722 62.115395) (end 56.206722 60.442395) (width 0.3) (layer "F.Cu") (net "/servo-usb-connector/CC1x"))
 (segment (start 59.331751 62.965395) (end 58.481751 62.115395) (width 0.3) (layer "F.Cu") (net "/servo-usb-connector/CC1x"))
 (segment (start 58.481751 62.115395) (end 57.879722 62.115395) (width 0.3) (layer "F.Cu") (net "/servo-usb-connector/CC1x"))
 (segment (start 56.206722 60.442395) (end 55.628251 60.442395) (width 0.3) (layer "F.Cu") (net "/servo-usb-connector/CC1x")))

